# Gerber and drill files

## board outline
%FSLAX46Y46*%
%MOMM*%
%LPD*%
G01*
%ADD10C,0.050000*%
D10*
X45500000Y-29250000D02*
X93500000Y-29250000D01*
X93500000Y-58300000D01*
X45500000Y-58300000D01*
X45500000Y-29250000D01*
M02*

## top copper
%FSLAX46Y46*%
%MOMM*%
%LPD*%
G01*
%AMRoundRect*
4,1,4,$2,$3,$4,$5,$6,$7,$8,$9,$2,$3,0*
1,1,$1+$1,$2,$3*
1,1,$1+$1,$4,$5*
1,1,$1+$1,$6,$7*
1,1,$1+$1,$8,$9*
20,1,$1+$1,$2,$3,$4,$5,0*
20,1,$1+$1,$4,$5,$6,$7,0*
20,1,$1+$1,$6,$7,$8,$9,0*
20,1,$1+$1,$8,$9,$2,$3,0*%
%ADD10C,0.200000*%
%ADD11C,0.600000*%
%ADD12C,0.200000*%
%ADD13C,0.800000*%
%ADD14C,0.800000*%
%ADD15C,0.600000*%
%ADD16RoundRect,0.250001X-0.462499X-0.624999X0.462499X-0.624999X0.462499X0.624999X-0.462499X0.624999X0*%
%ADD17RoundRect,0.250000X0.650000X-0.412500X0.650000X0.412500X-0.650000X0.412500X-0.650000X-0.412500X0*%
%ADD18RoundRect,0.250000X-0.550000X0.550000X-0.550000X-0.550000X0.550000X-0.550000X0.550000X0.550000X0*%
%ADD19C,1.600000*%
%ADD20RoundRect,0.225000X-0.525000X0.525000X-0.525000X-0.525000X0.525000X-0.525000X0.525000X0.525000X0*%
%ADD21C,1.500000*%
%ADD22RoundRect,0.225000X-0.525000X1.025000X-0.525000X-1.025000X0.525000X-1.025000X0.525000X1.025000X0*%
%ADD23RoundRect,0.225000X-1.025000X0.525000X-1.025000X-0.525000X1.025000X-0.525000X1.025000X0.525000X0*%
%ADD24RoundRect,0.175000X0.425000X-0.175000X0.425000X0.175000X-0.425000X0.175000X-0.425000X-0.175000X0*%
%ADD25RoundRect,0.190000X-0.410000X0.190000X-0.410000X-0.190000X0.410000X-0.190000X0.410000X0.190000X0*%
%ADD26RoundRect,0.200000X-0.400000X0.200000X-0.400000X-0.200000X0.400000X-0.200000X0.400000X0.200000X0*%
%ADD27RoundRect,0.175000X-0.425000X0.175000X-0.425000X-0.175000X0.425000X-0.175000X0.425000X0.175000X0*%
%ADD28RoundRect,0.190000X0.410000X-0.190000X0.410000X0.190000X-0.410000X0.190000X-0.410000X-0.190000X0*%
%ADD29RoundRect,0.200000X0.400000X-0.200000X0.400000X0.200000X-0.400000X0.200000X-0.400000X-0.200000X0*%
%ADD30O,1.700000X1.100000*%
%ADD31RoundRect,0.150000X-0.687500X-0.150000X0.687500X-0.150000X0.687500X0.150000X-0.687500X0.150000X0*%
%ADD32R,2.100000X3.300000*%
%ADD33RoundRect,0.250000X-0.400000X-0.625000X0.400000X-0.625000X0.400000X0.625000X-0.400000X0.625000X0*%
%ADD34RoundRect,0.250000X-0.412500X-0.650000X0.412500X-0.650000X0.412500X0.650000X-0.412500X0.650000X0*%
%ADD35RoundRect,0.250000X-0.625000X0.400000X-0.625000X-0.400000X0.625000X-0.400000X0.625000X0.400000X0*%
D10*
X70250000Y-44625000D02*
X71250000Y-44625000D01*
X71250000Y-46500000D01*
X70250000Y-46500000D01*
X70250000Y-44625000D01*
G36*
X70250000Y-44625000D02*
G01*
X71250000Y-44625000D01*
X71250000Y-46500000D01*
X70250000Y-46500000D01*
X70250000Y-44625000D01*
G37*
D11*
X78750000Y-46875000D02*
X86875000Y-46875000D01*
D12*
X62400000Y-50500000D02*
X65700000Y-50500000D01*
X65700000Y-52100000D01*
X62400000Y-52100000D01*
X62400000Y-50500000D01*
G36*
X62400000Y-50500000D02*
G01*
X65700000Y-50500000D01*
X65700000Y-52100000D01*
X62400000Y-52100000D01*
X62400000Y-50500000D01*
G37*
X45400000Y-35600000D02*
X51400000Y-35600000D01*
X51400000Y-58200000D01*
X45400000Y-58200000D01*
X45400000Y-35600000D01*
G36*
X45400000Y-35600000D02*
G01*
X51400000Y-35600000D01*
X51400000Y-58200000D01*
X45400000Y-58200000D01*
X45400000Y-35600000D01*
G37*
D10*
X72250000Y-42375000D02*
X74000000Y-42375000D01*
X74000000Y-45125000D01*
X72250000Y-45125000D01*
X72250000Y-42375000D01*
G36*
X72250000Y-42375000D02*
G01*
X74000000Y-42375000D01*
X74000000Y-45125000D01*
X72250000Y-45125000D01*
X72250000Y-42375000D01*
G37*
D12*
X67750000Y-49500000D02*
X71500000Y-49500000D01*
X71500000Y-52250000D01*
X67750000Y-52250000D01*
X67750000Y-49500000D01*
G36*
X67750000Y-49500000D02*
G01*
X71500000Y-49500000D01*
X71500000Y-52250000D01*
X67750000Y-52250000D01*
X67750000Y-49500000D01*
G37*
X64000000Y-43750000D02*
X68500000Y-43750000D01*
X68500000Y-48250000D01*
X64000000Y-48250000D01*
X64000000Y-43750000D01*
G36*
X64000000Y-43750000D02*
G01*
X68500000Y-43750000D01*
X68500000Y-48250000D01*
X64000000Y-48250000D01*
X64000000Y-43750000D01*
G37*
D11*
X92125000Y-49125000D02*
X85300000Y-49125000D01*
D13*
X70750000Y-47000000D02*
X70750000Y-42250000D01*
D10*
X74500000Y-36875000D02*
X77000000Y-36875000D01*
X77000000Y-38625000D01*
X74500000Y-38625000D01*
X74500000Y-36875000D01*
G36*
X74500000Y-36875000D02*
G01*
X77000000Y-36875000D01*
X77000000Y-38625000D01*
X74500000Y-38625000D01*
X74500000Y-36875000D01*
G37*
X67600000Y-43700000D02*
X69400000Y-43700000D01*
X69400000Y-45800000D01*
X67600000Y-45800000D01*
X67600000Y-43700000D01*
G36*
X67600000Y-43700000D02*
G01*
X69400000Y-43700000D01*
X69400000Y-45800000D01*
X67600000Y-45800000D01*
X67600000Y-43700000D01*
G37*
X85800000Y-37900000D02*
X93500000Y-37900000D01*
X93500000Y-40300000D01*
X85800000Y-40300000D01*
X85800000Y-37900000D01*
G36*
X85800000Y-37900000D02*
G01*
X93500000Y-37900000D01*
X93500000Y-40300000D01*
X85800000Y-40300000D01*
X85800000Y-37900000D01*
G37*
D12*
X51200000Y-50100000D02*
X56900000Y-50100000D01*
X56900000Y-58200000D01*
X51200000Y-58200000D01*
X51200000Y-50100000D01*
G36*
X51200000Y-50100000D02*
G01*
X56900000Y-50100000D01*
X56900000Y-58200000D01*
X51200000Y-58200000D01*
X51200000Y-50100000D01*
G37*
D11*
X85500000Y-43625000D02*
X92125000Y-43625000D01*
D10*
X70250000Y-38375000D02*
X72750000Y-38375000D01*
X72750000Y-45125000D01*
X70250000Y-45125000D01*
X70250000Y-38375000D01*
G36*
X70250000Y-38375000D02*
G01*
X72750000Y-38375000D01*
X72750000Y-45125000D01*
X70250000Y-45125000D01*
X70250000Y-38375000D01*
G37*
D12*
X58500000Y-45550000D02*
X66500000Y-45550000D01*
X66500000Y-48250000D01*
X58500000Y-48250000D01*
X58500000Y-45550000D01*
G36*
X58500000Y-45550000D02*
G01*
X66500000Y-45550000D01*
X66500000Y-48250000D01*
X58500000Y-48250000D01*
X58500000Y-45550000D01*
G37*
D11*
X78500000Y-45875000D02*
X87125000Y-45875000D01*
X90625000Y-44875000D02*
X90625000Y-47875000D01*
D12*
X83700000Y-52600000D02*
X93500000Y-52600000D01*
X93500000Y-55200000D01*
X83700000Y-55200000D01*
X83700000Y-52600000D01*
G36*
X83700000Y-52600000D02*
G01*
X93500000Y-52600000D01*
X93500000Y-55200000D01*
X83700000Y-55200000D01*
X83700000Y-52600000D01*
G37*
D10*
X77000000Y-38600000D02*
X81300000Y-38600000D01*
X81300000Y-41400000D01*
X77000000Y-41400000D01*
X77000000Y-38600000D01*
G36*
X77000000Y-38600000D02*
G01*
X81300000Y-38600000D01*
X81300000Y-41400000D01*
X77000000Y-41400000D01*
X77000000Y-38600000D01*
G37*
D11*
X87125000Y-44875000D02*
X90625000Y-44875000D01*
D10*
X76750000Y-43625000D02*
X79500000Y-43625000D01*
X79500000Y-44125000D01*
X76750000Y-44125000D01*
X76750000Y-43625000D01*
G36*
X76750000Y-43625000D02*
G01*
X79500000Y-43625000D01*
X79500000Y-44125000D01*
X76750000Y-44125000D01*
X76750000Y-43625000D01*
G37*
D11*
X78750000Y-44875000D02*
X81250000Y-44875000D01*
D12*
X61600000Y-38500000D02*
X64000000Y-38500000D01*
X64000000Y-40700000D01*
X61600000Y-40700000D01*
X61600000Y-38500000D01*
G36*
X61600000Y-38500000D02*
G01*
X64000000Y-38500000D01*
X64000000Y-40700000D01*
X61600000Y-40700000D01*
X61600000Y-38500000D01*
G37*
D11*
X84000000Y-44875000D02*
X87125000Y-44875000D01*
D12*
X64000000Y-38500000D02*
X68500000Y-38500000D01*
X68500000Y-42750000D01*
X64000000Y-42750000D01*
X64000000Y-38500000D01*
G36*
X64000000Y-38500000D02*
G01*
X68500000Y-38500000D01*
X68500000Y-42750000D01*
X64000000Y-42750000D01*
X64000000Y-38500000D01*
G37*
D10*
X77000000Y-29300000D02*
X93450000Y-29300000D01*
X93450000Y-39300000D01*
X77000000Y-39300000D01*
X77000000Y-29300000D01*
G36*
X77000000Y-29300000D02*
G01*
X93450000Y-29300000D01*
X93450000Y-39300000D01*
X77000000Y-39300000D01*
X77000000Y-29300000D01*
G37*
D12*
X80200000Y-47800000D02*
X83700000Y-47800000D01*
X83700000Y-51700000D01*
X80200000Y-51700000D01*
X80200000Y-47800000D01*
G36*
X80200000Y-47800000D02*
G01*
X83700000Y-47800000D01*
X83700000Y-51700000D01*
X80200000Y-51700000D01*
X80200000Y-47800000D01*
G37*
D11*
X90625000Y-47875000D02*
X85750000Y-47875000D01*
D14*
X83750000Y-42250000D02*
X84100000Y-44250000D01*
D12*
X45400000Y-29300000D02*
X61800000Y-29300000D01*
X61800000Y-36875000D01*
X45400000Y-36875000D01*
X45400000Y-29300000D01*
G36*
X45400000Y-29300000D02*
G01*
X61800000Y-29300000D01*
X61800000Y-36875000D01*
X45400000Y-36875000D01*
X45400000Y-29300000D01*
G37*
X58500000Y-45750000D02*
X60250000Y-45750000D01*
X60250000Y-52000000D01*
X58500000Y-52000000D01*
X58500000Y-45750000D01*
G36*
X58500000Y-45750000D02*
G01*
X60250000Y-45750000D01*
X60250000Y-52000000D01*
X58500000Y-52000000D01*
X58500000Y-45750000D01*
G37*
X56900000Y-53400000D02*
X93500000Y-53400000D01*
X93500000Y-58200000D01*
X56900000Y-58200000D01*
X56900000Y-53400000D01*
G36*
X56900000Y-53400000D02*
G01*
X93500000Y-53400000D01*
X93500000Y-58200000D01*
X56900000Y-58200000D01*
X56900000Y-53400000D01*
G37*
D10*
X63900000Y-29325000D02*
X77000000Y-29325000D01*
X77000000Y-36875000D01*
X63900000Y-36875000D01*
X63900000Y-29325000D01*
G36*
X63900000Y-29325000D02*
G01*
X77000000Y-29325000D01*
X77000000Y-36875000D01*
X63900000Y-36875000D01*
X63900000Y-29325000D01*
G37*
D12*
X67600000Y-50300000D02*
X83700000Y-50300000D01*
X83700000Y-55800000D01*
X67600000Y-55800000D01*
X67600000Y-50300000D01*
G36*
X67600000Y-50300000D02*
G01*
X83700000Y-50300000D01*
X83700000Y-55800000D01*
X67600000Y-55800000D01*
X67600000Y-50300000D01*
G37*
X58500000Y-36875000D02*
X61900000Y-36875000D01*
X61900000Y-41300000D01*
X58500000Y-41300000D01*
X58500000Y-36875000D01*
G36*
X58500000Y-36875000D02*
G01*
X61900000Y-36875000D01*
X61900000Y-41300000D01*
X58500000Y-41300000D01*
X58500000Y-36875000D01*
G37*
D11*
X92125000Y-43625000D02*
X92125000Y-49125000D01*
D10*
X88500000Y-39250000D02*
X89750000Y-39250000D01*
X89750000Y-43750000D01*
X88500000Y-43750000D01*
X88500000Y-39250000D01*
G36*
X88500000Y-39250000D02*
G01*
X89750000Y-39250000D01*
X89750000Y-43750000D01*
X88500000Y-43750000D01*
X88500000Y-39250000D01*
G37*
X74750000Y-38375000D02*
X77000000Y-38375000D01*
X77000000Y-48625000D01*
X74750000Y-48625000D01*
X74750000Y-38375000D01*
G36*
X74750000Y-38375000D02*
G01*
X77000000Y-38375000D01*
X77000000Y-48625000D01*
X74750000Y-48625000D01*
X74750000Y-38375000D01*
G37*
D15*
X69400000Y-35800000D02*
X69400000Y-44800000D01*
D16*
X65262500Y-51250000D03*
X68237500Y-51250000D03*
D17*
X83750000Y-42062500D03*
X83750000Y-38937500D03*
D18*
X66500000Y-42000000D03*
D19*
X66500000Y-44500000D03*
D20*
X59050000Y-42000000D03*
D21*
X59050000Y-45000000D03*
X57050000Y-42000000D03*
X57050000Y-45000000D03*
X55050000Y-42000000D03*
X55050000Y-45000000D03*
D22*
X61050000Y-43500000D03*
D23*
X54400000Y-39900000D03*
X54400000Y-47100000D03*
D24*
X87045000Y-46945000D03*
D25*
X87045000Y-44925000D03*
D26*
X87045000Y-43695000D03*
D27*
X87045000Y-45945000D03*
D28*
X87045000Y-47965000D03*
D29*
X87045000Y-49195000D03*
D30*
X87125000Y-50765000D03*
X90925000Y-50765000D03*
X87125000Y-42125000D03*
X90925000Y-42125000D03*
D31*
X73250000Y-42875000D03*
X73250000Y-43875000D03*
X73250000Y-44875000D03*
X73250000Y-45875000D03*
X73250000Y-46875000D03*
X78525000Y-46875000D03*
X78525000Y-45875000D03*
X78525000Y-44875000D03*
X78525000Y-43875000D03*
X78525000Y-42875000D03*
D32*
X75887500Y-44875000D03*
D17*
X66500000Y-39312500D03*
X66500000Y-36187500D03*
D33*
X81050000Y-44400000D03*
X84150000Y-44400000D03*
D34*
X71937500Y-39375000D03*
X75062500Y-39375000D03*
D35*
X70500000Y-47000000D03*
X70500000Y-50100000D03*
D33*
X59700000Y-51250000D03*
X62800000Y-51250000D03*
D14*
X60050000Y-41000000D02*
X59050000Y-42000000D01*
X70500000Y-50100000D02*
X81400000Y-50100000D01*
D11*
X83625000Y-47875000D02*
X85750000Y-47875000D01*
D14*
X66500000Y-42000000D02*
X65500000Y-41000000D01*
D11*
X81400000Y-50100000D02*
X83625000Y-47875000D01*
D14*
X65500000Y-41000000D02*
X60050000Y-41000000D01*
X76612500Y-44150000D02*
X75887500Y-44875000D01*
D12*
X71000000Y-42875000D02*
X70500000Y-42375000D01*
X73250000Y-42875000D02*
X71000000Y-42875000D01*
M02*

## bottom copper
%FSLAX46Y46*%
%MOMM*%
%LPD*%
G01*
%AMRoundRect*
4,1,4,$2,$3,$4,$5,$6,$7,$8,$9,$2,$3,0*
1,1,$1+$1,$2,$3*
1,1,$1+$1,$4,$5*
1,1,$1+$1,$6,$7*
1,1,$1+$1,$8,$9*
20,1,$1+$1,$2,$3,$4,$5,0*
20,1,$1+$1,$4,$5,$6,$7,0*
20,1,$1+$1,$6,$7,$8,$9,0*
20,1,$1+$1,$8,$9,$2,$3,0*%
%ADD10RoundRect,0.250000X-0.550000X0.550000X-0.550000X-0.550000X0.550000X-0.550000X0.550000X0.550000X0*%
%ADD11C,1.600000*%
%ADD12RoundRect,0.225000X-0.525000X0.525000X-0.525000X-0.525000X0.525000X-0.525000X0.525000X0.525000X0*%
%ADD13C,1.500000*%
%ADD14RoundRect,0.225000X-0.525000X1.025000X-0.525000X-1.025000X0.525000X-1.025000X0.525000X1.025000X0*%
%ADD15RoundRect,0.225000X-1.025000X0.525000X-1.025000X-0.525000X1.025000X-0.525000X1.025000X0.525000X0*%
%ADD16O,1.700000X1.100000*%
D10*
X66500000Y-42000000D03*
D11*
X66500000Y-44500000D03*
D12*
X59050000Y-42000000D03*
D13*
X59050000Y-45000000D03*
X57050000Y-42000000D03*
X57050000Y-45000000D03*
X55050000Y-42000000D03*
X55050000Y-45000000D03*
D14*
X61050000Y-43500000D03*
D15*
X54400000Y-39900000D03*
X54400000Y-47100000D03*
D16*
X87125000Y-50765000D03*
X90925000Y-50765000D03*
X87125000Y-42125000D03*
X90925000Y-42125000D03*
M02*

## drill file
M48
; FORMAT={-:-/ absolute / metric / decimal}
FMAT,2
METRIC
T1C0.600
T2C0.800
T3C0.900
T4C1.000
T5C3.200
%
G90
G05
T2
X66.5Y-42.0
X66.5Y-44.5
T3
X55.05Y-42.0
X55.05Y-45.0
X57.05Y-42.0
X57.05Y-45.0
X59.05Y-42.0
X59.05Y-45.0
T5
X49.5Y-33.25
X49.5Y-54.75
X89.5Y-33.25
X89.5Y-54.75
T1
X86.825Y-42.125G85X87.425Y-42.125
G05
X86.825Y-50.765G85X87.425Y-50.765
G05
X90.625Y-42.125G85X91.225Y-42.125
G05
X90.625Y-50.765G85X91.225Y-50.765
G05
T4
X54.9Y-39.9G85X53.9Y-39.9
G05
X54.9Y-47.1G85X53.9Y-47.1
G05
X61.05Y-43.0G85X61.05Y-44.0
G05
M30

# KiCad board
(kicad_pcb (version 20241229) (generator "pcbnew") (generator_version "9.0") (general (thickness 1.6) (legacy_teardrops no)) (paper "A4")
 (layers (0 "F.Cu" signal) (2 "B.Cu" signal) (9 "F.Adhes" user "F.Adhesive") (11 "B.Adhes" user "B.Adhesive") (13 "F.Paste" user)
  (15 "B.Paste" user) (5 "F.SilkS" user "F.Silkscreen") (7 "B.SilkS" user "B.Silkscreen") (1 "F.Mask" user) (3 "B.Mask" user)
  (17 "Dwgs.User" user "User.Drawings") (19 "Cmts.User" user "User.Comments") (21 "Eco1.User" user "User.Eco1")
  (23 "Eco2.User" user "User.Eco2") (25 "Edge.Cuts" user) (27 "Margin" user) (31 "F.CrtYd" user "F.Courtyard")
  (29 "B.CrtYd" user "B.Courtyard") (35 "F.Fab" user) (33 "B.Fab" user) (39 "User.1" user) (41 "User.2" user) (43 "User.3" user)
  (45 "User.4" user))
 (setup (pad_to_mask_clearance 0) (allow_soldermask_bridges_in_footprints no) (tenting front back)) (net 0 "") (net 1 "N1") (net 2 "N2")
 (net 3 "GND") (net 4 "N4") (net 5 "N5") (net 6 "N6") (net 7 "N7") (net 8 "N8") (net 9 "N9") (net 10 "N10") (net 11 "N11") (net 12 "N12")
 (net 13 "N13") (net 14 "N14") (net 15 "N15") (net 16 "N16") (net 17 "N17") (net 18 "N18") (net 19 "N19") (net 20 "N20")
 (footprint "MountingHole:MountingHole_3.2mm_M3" (layer "F.Cu") (at 89.5 54.75)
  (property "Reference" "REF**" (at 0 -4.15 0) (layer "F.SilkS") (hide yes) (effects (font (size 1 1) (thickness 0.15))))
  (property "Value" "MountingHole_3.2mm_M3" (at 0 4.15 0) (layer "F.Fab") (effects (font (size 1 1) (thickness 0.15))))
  (pad "" np_thru_hole circle (at 0 0) (size 3.2 3.2) (drill 3.2) (layers "*.Cu" "*.Mask")))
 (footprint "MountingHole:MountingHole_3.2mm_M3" (layer "F.Cu") (at 49.5 33.25)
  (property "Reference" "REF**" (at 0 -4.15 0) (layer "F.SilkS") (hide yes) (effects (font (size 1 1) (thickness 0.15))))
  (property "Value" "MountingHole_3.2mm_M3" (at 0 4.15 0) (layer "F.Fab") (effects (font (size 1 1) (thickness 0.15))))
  (pad "" np_thru_hole circle (at 0 0) (size 3.2 3.2) (drill 3.2) (layers "*.Cu" "*.Mask")))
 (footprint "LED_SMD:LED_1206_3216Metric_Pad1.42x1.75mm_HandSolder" (layer "F.Cu") (at 66.75 51.25)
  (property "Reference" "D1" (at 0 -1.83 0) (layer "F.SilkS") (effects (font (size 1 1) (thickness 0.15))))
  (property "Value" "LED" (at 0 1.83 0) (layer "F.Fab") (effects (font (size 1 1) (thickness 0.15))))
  (pad "1" smd roundrect (at -1.4875 0) (size 1.425 1.75) (layers "F.Cu" "F.Mask" "F.Paste") (roundrect_rratio 0.175439) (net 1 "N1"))
  (pad "2" smd roundrect (at 1.4875 0) (size 1.425 1.75) (layers "F.Cu" "F.Mask" "F.Paste") (roundrect_rratio 0.175439) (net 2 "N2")))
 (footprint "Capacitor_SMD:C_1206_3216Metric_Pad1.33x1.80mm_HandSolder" (layer "F.Cu") (at 83.75 40.5 90)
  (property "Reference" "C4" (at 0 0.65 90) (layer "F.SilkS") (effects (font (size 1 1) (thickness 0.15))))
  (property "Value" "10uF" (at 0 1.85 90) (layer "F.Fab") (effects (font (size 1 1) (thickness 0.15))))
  (pad "1" smd roundrect (at -1.5625 0 90) (size 1.325 1.8) (layers "F.Cu" "F.Mask" "F.Paste") (roundrect_rratio 0.188679) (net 2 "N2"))
  (pad "2" smd roundrect (at 1.5625 0 90) (size 1.325 1.8) (layers "F.Cu" "F.Mask" "F.Paste") (roundrect_rratio 0.188679) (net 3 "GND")))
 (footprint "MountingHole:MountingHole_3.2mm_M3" (layer "F.Cu") (at 89.5 33.25)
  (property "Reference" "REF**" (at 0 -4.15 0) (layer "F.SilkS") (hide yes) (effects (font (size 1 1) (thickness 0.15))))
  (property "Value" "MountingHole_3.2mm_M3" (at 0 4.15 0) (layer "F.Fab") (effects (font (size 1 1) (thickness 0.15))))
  (pad "" np_thru_hole circle (at 0 0) (size 3.2 3.2) (drill 3.2) (layers "*.Cu" "*.Mask")))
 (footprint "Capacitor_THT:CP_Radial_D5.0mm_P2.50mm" (layer "F.Cu") (at 66.5 42 -90)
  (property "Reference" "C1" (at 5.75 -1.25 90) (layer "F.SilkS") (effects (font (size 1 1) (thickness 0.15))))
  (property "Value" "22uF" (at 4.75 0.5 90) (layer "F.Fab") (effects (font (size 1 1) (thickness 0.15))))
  (pad "1" thru_hole roundrect (at 0 0 270) (size 1.6 1.6) (drill 0.8) (layers "*.Cu" "*.Mask") (remove_unused_layers no)
   (roundrect_rratio 0.15625) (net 2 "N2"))
  (pad "2" thru_hole circle (at 2.5 0 270) (size 1.6 1.6) (drill 0.8) (layers "*.Cu" "*.Mask") (remove_unused_layers no) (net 3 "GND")))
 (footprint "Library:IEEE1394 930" (layer "F.Cu") (at 45.5 43.5 -90)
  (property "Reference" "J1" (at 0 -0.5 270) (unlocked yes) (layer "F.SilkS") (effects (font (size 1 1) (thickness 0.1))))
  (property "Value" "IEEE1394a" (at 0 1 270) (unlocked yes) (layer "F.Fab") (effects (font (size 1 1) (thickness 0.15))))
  (pad "1" thru_hole roundrect (at -1.5 -13.55 270) (size 1.5 1.5) (drill 0.9) (layers "*.Cu" "*.Mask") (remove_unused_layers no)
   (roundrect_rratio 0.15) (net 2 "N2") (thermal_bridge_angle 45))
  (pad "2" thru_hole circle (at 1.5 -13.55 270) (size 1.5 1.5) (drill 0.9) (layers "*.Cu" "*.Mask") (remove_unused_layers no) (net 3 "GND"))
  (pad "3" thru_hole circle (at -1.5 -11.55 270) (size 1.5 1.5) (drill 0.9) (layers "*.Cu" "*.Mask") (remove_unused_layers no) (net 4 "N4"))
  (pad "4" thru_hole circle (at 1.5 -11.55 270) (size 1.5 1.5) (drill 0.9) (layers "*.Cu" "*.Mask") (remove_unused_layers no) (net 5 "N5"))
  (pad "5" thru_hole circle (at -1.5 -9.55 270) (size 1.5 1.5) (drill 0.9) (layers "*.Cu" "*.Mask") (remove_unused_layers no) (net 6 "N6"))
  (pad "6" thru_hole circle (at 1.5 -9.55 270) (size 1.5 1.5) (drill 0.9) (layers "*.Cu" "*.Mask") (remove_unused_layers no) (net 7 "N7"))
  (pad "7" thru_hole roundrect (at 0 -15.55 270) (size 2.5 1.5) (drill oval 2 1) (layers "*.Cu" "*.Mask") (remove_unused_layers no)
   (roundrect_rratio 0.15) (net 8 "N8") (thermal_bridge_angle 45))
  (pad "8" thru_hole roundrect (at -3.6 -8.9 270) (size 1.5 2.5) (drill oval 1 2) (layers "*.Cu" "*.Mask") (remove_unused_layers no)
   (roundrect_rratio 0.15) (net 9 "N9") (thermal_bridge_angle 45))
  (pad "9" thru_hole roundrect (at 3.6 -8.9 270) (size 1.5 2.5) (drill oval 1 2) (layers "*.Cu" "*.Mask") (remove_unused_layers no)
   (roundrect_rratio 0.15) (thermal_bridge_angle 45)))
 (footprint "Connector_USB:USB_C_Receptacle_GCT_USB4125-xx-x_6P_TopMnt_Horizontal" (layer "F.Cu") (at 90.125 46.445 90)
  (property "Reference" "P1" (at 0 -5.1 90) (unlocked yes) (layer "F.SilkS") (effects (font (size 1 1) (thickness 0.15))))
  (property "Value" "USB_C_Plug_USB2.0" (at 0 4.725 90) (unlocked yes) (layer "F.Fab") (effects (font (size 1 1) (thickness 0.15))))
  (pad "A5" smd roundrect (at -0.5 -3.08 90) (size 0.7 1.2) (layers "F.Cu" "F.Mask" "F.Paste") (roundrect_rratio 0.25) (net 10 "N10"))
  (pad "A9" smd roundrect (at 1.52 -3.08 270) (size 0.76 1.2) (layers "F.Cu" "F.Mask" "F.Paste") (roundrect_rratio 0.25) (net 2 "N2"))
  (pad "A12" smd roundrect (at 2.75 -3.08 270) (size 0.8 1.2) (layers "F.Cu" "F.Mask" "F.Paste") (roundrect_rratio 0.25) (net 3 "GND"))
  (pad "B5" smd roundrect (at 0.5 -3.08 270) (size 0.7 1.2) (layers "F.Cu" "F.Mask" "F.Paste") (roundrect_rratio 0.25) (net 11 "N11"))
  (pad "B9" smd roundrect (at -1.52 -3.08 90) (size 0.76 1.2) (layers "F.Cu" "F.Mask" "F.Paste") (roundrect_rratio 0.25) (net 2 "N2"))
  (pad "B12" smd roundrect (at -2.75 -3.08 90) (size 0.8 1.2) (layers "F.Cu" "F.Mask" "F.Paste") (roundrect_rratio 0.25) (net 3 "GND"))
  (pad "S1" thru_hole oval (at -4.32 -3 90) (size 1.1 1.7) (drill oval 0.6 1.2) (layers "*.Cu" "*.Mask" "F.Paste") (remove_unused_layers no)
   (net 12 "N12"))
  (pad "S1" thru_hole oval (at -4.32 0.8 90) (size 1.1 1.7) (drill oval 0.6 1.2) (layers "*.Cu" "*.Mask" "F.Paste")
   (remove_unused_layers no) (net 12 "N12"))
  (pad "S1" thru_hole oval (at 4.32 -3 90) (size 1.1 1.7) (drill oval 0.6 1.2) (layers "*.Cu" "*.Mask" "F.Paste") (remove_unused_layers no)
   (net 12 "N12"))
  (pad "S1" thru_hole oval (at 4.32 0.8 90) (size 1.1 1.7) (drill oval 0.6 1.2) (layers "*.Cu" "*.Mask" "F.Paste") (remove_unused_layers no)
   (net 12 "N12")))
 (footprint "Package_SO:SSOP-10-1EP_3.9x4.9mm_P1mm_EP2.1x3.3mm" (layer "F.Cu") (at 75.8875 44.875)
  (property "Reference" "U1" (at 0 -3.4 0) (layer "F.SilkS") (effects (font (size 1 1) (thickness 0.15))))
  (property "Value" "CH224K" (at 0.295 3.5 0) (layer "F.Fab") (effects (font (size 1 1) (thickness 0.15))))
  (pad "" smd roundrect (at 0 0) (size 1.69 2.66) (layers "F.Paste") (roundrect_rratio 0.147929))
  (pad "1" smd roundrect (at -2.6375 -2) (size 1.675 0.6) (layers "F.Cu" "F.Mask" "F.Paste") (roundrect_rratio 0.25) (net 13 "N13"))
  (pad "2" smd roundrect (at -2.6375 -1) (size 1.675 0.6) (layers "F.Cu" "F.Mask" "F.Paste") (roundrect_rratio 0.25) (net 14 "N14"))
  (pad "3" smd roundrect (at -2.6375 0) (size 1.675 0.6) (layers "F.Cu" "F.Mask" "F.Paste") (roundrect_rratio 0.25) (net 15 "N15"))
  (pad "4" smd roundrect (at -2.6375 1) (size 1.675 0.6) (layers "F.Cu" "F.Mask" "F.Paste") (roundrect_rratio 0.25) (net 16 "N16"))
  (pad "5" smd roundrect (at -2.6375 2) (size 1.675 0.6) (layers "F.Cu" "F.Mask" "F.Paste") (roundrect_rratio 0.25) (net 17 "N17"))
  (pad "6" smd roundrect (at 2.6375 2) (size 1.675 0.6) (layers "F.Cu" "F.Mask" "F.Paste") (roundrect_rratio 0.25) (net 10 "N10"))
  (pad "7" smd roundrect (at 2.6375 1) (size 1.675 0.6) (layers "F.Cu" "F.Mask" "F.Paste") (roundrect_rratio 0.25) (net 10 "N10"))
  (pad "8" smd roundrect (at 2.6375 0) (size 1.675 0.6) (layers "F.Cu" "F.Mask" "F.Paste") (roundrect_rratio 0.25) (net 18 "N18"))
  (pad "9" smd roundrect (at 2.6375 -1) (size 1.675 0.6) (layers "F.Cu" "F.Mask" "F.Paste") (roundrect_rratio 0.25) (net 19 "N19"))
  (pad "10" smd roundrect (at 2.6375 -2) (size 1.675 0.6) (layers "F.Cu" "F.Mask" "F.Paste") (roundrect_rratio 0.25) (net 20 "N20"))
  (pad "11" smd rect (at 0 0) (size 2.1 3.3) (layers "F.Cu" "F.Mask") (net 3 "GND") (zone_connect 2)))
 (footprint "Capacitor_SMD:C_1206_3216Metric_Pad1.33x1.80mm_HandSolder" (layer "F.Cu") (at 66.5 37.75 90)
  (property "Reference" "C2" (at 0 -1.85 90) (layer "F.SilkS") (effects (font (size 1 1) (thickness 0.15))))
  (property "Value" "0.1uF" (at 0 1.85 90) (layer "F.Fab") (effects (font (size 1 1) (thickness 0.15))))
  (pad "1" smd roundrect (at -1.5625 0 90) (size 1.325 1.8) (layers "F.Cu" "F.Mask" "F.Paste") (roundrect_rratio 0.188679) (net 2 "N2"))
  (pad "2" smd roundrect (at 1.5625 0 90) (size 1.325 1.8) (layers "F.Cu" "F.Mask" "F.Paste") (roundrect_rratio 0.188679) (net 3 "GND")))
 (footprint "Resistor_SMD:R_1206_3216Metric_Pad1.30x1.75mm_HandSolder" (layer "F.Cu") (at 82.6 44.4)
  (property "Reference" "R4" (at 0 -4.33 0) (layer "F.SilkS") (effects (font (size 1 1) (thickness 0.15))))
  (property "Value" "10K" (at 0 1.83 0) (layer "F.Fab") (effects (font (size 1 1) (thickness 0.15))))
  (pad "1" smd roundrect (at -1.55 0) (size 1.3 1.75) (layers "F.Cu" "F.Mask" "F.Paste") (roundrect_rratio 0.192308) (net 18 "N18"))
  (pad "2" smd roundrect (at 1.55 0) (size 1.3 1.75) (layers "F.Cu" "F.Mask" "F.Paste") (roundrect_rratio 0.192308) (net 2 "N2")))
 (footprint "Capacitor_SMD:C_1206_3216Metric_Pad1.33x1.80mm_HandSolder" (layer "F.Cu") (at 73.5 39.375)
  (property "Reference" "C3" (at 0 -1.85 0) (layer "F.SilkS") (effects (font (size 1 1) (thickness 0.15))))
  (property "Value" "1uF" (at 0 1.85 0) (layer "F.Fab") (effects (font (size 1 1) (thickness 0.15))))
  (pad "1" smd roundrect (at -1.5625 0) (size 1.325 1.8) (layers "F.Cu" "F.Mask" "F.Paste") (roundrect_rratio 0.188679) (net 13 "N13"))
  (pad "2" smd roundrect (at 1.5625 0) (size 1.325 1.8) (layers "F.Cu" "F.Mask" "F.Paste") (roundrect_rratio 0.188679) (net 3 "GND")))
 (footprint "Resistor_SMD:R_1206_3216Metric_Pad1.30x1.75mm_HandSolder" (layer "F.Cu") (at 70.5 48.55 -90)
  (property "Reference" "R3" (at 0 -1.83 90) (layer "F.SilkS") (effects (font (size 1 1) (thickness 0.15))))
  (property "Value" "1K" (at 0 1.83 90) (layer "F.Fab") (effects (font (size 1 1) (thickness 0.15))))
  (pad "1" smd roundrect (at -1.55 0 270) (size 1.3 1.75) (layers "F.Cu" "F.Mask" "F.Paste") (roundrect_rratio 0.192308) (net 13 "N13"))
  (pad "2" smd roundrect (at 1.55 0 270) (size 1.3 1.75) (layers "F.Cu" "F.Mask" "F.Paste") (roundrect_rratio 0.192308) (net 2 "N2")))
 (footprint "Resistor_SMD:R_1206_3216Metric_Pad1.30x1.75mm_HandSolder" (layer "F.Cu") (at 61.25 51.25)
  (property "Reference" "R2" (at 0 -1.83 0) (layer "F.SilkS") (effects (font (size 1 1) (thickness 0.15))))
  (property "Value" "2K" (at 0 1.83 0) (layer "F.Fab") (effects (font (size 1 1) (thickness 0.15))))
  (pad "1" smd roundrect (at -1.55 0) (size 1.3 1.75) (layers "F.Cu" "F.Mask" "F.Paste") (roundrect_rratio 0.192308) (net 3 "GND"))
  (pad "2" smd roundrect (at 1.55 0) (size 1.3 1.75) (layers "F.Cu" "F.Mask" "F.Paste") (roundrect_rratio 0.192308) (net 1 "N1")))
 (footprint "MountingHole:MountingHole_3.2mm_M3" (layer "F.Cu") (at 49.5 54.75)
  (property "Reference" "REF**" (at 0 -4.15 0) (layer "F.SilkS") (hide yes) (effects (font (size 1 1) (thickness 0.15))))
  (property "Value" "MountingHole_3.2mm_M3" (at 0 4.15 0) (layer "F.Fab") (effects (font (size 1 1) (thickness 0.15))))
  (pad "" np_thru_hole circle (at 0 0) (size 3.2 3.2) (drill 3.2) (layers "*.Cu" "*.Mask")))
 (gr_rect (start 70.25 44.625) (end 71.25 46.5) (stroke (width 0.2) (type solid)) (fill yes) (layer "F.Cu"))
 (gr_line (start 78.75 46.875) (end 86.875 46.875) (stroke (width 0.6) (type solid)) (layer "F.Cu") (net 10))
 (gr_rect (start 62.4 50.5) (end 65.7 52.1) (stroke (width 0.2) (type solid)) (fill yes) (layer "F.Cu") (net 1))
 (gr_rect (start 45.4 35.6) (end 51.4 58.2) (stroke (width 0.2) (type solid)) (fill yes) (layer "F.Cu") (net 2))
 (gr_rect (start 72.25 42.375) (end 74 45.125) (stroke (width 0.2) (type solid)) (fill yes) (layer "F.Cu"))
 (gr_rect (start 67.75 49.5) (end 71.5 52.25) (stroke (width 0.2) (type solid)) (fill yes) (layer "F.Cu") (net 2))
 (gr_rect (start 64 43.75) (end 68.5 48.25) (stroke (width 0.2) (type solid)) (fill yes) (layer "F.Cu") (net 3))
 (gr_line (start 92.125 49.125) (end 85.3 49.125) (stroke (width 0.6) (type solid)) (layer "F.Cu") (net 3))
 (gr_line (start 70.75 47) (end 70.75 42.25) (stroke (width 0.8) (type solid)) (layer "F.Cu"))
 (gr_rect (start 74.5 36.875) (end 77 38.625) (stroke (width 0.2) (type solid)) (fill yes) (layer "F.Cu"))
 (gr_rect (start 67.6 43.7) (end 69.4 45.8) (stroke (width 0.2) (type solid)) (fill yes) (layer "F.Cu"))
 (gr_rect (start 85.8 37.9) (end 93.5 40.3) (stroke (width 0.2) (type solid)) (fill yes) (layer "F.Cu"))
 (gr_rect (start 51.2 50.1) (end 56.9 58.2) (stroke (width 0.2) (type solid)) (fill yes) (layer "F.Cu") (net 2))
 (gr_line (start 85.5 43.625) (end 92.125 43.625) (stroke (width 0.6) (type solid)) (layer "F.Cu") (net 3))
 (gr_rect (start 70.25 38.375) (end 72.75 45.125) (stroke (width 0.2) (type solid)) (fill yes) (layer "F.Cu"))
 (gr_rect (start 58.5 45.55) (end 66.5 48.25) (stroke (width 0.2) (type solid)) (fill yes) (layer "F.Cu") (net 3))
 (gr_line (start 78.5 45.875) (end 87.125 45.875) (stroke (width 0.6) (type solid)) (layer "F.Cu") (net 11))
 (gr_line (start 90.625 44.875) (end 90.625 47.875) (stroke (width 0.6) (type solid)) (layer "F.Cu") (net 2))
 (gr_rect (start 83.7 52.6) (end 93.5 55.2) (stroke (width 0.2) (type solid)) (fill yes) (layer "F.Cu") (net 2))
 (gr_rect (start 77 38.6) (end 81.3 41.4) (stroke (width 0.2) (type solid)) (fill yes) (layer "F.Cu"))
 (gr_line (start 87.125 44.875) (end 90.625 44.875) (stroke (width 0.6) (type solid)) (layer "F.Cu") (net 2))
 (gr_rect (start 76.75 43.625) (end 79.5 44.125) (stroke (width 0.2) (type solid)) (fill yes) (layer "F.Cu"))
 (gr_line (start 78.75 44.875) (end 81.25 44.875) (stroke (width 0.6) (type solid)) (layer "F.Cu") (net 18))
 (gr_rect (start 61.6 38.5) (end 64 40.7) (stroke (width 0.2) (type solid)) (fill yes) (layer "F.Cu") (net 2))
 (gr_line (start 84 44.875) (end 87.125 44.875) (stroke (width 0.6) (type solid)) (layer "F.Cu") (net 2))
 (gr_rect (start 64 38.5) (end 68.5 42.75) (stroke (width 0.2) (type solid)) (fill yes) (layer "F.Cu") (net 2))
 (gr_rect (start 77 29.3) (end 93.45 39.3) (stroke (width 0.2) (type solid)) (fill yes) (layer "F.Cu"))
 (gr_rect (start 80.2 47.8) (end 83.7 51.7) (stroke (width 0.2) (type solid)) (fill yes) (layer "F.Cu") (net 2))
 (gr_line (start 90.625 47.875) (end 85.75 47.875) (stroke (width 0.6) (type solid)) (layer "F.Cu") (net 2))
 (gr_line (start 83.75 42.25) (end 84.1 44.25) (stroke (width 0.8) (type solid)) (layer "F.Cu") (net 2))
 (gr_rect (start 45.4 29.3) (end 61.8 36.875) (stroke (width 0.2) (type solid)) (fill yes) (layer "F.Cu") (net 2))
 (gr_rect (start 58.5 45.75) (end 60.25 52) (stroke (width 0.2) (type solid)) (fill yes) (layer "F.Cu") (net 3))
 (gr_rect (start 56.9 53.4) (end 93.5 58.2) (stroke (width 0.2) (type solid)) (fill yes) (layer "F.Cu") (net 2))
 (gr_rect (start 63.9 29.325) (end 77 36.875) (stroke (width 0.2) (type solid)) (fill yes) (layer "F.Cu"))
 (gr_rect (start 67.6 50.3) (end 83.7 55.8) (stroke (width 0.2) (type solid)) (fill yes) (layer "F.Cu") (net 2))
 (gr_rect (start 58.5 36.875) (end 61.9 41.3) (stroke (width 0.2) (type solid)) (fill yes) (layer "F.Cu") (net 2))
 (gr_line (start 92.125 43.625) (end 92.125 49.125) (stroke (width 0.6) (type solid)) (layer "F.Cu") (net 3))
 (gr_rect (start 88.5 39.25) (end 89.75 43.75) (stroke (width 0.2) (type solid)) (fill yes) (layer "F.Cu"))
 (gr_rect (start 74.75 38.375) (end 77 48.625) (stroke (width 0.2) (type solid)) (fill yes) (layer "F.Cu"))
 (gr_line (start 69.4 35.8) (end 69.4 44.8) (stroke (width 0.6) (type solid)) (layer "F.Cu"))
 (gr_rect (start 45.5 29.25) (end 93.5 58.3) (stroke (width 0.05) (type default)) (fill no) (layer "Edge.Cuts"))
 (segment (start 60.05 41) (end 59.05 42) (width 0.8) (layer "F.Cu") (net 2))
 (segment (start 70.5 50.1) (end 81.4 50.1) (width 0.8) (layer "F.Cu") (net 2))
 (segment (start 83.625 47.875) (end 85.75 47.875) (width 0.6) (layer "F.Cu") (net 2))
 (segment (start 66.5 42) (end 65.5 41) (width 0.8) (layer "F.Cu") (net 2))
 (segment (start 81.4 50.1) (end 83.625 47.875) (width 0.6) (layer "F.Cu") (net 2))
 (segment (start 65.5 41) (end 60.05 41) (width 0.8) (layer "F.Cu") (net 2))
 (segment (start 76.6125 44.15) (end 75.8875 44.875) (width 0.8) (layer "F.Cu") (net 3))
 (segment (start 71 42.875) (end 70.5 42.375) (width 0.2) (layer "F.Cu") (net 13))
 (segment (start 73.25 42.875) (end 71 42.875) (width 0.2) (layer "F.Cu") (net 13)))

